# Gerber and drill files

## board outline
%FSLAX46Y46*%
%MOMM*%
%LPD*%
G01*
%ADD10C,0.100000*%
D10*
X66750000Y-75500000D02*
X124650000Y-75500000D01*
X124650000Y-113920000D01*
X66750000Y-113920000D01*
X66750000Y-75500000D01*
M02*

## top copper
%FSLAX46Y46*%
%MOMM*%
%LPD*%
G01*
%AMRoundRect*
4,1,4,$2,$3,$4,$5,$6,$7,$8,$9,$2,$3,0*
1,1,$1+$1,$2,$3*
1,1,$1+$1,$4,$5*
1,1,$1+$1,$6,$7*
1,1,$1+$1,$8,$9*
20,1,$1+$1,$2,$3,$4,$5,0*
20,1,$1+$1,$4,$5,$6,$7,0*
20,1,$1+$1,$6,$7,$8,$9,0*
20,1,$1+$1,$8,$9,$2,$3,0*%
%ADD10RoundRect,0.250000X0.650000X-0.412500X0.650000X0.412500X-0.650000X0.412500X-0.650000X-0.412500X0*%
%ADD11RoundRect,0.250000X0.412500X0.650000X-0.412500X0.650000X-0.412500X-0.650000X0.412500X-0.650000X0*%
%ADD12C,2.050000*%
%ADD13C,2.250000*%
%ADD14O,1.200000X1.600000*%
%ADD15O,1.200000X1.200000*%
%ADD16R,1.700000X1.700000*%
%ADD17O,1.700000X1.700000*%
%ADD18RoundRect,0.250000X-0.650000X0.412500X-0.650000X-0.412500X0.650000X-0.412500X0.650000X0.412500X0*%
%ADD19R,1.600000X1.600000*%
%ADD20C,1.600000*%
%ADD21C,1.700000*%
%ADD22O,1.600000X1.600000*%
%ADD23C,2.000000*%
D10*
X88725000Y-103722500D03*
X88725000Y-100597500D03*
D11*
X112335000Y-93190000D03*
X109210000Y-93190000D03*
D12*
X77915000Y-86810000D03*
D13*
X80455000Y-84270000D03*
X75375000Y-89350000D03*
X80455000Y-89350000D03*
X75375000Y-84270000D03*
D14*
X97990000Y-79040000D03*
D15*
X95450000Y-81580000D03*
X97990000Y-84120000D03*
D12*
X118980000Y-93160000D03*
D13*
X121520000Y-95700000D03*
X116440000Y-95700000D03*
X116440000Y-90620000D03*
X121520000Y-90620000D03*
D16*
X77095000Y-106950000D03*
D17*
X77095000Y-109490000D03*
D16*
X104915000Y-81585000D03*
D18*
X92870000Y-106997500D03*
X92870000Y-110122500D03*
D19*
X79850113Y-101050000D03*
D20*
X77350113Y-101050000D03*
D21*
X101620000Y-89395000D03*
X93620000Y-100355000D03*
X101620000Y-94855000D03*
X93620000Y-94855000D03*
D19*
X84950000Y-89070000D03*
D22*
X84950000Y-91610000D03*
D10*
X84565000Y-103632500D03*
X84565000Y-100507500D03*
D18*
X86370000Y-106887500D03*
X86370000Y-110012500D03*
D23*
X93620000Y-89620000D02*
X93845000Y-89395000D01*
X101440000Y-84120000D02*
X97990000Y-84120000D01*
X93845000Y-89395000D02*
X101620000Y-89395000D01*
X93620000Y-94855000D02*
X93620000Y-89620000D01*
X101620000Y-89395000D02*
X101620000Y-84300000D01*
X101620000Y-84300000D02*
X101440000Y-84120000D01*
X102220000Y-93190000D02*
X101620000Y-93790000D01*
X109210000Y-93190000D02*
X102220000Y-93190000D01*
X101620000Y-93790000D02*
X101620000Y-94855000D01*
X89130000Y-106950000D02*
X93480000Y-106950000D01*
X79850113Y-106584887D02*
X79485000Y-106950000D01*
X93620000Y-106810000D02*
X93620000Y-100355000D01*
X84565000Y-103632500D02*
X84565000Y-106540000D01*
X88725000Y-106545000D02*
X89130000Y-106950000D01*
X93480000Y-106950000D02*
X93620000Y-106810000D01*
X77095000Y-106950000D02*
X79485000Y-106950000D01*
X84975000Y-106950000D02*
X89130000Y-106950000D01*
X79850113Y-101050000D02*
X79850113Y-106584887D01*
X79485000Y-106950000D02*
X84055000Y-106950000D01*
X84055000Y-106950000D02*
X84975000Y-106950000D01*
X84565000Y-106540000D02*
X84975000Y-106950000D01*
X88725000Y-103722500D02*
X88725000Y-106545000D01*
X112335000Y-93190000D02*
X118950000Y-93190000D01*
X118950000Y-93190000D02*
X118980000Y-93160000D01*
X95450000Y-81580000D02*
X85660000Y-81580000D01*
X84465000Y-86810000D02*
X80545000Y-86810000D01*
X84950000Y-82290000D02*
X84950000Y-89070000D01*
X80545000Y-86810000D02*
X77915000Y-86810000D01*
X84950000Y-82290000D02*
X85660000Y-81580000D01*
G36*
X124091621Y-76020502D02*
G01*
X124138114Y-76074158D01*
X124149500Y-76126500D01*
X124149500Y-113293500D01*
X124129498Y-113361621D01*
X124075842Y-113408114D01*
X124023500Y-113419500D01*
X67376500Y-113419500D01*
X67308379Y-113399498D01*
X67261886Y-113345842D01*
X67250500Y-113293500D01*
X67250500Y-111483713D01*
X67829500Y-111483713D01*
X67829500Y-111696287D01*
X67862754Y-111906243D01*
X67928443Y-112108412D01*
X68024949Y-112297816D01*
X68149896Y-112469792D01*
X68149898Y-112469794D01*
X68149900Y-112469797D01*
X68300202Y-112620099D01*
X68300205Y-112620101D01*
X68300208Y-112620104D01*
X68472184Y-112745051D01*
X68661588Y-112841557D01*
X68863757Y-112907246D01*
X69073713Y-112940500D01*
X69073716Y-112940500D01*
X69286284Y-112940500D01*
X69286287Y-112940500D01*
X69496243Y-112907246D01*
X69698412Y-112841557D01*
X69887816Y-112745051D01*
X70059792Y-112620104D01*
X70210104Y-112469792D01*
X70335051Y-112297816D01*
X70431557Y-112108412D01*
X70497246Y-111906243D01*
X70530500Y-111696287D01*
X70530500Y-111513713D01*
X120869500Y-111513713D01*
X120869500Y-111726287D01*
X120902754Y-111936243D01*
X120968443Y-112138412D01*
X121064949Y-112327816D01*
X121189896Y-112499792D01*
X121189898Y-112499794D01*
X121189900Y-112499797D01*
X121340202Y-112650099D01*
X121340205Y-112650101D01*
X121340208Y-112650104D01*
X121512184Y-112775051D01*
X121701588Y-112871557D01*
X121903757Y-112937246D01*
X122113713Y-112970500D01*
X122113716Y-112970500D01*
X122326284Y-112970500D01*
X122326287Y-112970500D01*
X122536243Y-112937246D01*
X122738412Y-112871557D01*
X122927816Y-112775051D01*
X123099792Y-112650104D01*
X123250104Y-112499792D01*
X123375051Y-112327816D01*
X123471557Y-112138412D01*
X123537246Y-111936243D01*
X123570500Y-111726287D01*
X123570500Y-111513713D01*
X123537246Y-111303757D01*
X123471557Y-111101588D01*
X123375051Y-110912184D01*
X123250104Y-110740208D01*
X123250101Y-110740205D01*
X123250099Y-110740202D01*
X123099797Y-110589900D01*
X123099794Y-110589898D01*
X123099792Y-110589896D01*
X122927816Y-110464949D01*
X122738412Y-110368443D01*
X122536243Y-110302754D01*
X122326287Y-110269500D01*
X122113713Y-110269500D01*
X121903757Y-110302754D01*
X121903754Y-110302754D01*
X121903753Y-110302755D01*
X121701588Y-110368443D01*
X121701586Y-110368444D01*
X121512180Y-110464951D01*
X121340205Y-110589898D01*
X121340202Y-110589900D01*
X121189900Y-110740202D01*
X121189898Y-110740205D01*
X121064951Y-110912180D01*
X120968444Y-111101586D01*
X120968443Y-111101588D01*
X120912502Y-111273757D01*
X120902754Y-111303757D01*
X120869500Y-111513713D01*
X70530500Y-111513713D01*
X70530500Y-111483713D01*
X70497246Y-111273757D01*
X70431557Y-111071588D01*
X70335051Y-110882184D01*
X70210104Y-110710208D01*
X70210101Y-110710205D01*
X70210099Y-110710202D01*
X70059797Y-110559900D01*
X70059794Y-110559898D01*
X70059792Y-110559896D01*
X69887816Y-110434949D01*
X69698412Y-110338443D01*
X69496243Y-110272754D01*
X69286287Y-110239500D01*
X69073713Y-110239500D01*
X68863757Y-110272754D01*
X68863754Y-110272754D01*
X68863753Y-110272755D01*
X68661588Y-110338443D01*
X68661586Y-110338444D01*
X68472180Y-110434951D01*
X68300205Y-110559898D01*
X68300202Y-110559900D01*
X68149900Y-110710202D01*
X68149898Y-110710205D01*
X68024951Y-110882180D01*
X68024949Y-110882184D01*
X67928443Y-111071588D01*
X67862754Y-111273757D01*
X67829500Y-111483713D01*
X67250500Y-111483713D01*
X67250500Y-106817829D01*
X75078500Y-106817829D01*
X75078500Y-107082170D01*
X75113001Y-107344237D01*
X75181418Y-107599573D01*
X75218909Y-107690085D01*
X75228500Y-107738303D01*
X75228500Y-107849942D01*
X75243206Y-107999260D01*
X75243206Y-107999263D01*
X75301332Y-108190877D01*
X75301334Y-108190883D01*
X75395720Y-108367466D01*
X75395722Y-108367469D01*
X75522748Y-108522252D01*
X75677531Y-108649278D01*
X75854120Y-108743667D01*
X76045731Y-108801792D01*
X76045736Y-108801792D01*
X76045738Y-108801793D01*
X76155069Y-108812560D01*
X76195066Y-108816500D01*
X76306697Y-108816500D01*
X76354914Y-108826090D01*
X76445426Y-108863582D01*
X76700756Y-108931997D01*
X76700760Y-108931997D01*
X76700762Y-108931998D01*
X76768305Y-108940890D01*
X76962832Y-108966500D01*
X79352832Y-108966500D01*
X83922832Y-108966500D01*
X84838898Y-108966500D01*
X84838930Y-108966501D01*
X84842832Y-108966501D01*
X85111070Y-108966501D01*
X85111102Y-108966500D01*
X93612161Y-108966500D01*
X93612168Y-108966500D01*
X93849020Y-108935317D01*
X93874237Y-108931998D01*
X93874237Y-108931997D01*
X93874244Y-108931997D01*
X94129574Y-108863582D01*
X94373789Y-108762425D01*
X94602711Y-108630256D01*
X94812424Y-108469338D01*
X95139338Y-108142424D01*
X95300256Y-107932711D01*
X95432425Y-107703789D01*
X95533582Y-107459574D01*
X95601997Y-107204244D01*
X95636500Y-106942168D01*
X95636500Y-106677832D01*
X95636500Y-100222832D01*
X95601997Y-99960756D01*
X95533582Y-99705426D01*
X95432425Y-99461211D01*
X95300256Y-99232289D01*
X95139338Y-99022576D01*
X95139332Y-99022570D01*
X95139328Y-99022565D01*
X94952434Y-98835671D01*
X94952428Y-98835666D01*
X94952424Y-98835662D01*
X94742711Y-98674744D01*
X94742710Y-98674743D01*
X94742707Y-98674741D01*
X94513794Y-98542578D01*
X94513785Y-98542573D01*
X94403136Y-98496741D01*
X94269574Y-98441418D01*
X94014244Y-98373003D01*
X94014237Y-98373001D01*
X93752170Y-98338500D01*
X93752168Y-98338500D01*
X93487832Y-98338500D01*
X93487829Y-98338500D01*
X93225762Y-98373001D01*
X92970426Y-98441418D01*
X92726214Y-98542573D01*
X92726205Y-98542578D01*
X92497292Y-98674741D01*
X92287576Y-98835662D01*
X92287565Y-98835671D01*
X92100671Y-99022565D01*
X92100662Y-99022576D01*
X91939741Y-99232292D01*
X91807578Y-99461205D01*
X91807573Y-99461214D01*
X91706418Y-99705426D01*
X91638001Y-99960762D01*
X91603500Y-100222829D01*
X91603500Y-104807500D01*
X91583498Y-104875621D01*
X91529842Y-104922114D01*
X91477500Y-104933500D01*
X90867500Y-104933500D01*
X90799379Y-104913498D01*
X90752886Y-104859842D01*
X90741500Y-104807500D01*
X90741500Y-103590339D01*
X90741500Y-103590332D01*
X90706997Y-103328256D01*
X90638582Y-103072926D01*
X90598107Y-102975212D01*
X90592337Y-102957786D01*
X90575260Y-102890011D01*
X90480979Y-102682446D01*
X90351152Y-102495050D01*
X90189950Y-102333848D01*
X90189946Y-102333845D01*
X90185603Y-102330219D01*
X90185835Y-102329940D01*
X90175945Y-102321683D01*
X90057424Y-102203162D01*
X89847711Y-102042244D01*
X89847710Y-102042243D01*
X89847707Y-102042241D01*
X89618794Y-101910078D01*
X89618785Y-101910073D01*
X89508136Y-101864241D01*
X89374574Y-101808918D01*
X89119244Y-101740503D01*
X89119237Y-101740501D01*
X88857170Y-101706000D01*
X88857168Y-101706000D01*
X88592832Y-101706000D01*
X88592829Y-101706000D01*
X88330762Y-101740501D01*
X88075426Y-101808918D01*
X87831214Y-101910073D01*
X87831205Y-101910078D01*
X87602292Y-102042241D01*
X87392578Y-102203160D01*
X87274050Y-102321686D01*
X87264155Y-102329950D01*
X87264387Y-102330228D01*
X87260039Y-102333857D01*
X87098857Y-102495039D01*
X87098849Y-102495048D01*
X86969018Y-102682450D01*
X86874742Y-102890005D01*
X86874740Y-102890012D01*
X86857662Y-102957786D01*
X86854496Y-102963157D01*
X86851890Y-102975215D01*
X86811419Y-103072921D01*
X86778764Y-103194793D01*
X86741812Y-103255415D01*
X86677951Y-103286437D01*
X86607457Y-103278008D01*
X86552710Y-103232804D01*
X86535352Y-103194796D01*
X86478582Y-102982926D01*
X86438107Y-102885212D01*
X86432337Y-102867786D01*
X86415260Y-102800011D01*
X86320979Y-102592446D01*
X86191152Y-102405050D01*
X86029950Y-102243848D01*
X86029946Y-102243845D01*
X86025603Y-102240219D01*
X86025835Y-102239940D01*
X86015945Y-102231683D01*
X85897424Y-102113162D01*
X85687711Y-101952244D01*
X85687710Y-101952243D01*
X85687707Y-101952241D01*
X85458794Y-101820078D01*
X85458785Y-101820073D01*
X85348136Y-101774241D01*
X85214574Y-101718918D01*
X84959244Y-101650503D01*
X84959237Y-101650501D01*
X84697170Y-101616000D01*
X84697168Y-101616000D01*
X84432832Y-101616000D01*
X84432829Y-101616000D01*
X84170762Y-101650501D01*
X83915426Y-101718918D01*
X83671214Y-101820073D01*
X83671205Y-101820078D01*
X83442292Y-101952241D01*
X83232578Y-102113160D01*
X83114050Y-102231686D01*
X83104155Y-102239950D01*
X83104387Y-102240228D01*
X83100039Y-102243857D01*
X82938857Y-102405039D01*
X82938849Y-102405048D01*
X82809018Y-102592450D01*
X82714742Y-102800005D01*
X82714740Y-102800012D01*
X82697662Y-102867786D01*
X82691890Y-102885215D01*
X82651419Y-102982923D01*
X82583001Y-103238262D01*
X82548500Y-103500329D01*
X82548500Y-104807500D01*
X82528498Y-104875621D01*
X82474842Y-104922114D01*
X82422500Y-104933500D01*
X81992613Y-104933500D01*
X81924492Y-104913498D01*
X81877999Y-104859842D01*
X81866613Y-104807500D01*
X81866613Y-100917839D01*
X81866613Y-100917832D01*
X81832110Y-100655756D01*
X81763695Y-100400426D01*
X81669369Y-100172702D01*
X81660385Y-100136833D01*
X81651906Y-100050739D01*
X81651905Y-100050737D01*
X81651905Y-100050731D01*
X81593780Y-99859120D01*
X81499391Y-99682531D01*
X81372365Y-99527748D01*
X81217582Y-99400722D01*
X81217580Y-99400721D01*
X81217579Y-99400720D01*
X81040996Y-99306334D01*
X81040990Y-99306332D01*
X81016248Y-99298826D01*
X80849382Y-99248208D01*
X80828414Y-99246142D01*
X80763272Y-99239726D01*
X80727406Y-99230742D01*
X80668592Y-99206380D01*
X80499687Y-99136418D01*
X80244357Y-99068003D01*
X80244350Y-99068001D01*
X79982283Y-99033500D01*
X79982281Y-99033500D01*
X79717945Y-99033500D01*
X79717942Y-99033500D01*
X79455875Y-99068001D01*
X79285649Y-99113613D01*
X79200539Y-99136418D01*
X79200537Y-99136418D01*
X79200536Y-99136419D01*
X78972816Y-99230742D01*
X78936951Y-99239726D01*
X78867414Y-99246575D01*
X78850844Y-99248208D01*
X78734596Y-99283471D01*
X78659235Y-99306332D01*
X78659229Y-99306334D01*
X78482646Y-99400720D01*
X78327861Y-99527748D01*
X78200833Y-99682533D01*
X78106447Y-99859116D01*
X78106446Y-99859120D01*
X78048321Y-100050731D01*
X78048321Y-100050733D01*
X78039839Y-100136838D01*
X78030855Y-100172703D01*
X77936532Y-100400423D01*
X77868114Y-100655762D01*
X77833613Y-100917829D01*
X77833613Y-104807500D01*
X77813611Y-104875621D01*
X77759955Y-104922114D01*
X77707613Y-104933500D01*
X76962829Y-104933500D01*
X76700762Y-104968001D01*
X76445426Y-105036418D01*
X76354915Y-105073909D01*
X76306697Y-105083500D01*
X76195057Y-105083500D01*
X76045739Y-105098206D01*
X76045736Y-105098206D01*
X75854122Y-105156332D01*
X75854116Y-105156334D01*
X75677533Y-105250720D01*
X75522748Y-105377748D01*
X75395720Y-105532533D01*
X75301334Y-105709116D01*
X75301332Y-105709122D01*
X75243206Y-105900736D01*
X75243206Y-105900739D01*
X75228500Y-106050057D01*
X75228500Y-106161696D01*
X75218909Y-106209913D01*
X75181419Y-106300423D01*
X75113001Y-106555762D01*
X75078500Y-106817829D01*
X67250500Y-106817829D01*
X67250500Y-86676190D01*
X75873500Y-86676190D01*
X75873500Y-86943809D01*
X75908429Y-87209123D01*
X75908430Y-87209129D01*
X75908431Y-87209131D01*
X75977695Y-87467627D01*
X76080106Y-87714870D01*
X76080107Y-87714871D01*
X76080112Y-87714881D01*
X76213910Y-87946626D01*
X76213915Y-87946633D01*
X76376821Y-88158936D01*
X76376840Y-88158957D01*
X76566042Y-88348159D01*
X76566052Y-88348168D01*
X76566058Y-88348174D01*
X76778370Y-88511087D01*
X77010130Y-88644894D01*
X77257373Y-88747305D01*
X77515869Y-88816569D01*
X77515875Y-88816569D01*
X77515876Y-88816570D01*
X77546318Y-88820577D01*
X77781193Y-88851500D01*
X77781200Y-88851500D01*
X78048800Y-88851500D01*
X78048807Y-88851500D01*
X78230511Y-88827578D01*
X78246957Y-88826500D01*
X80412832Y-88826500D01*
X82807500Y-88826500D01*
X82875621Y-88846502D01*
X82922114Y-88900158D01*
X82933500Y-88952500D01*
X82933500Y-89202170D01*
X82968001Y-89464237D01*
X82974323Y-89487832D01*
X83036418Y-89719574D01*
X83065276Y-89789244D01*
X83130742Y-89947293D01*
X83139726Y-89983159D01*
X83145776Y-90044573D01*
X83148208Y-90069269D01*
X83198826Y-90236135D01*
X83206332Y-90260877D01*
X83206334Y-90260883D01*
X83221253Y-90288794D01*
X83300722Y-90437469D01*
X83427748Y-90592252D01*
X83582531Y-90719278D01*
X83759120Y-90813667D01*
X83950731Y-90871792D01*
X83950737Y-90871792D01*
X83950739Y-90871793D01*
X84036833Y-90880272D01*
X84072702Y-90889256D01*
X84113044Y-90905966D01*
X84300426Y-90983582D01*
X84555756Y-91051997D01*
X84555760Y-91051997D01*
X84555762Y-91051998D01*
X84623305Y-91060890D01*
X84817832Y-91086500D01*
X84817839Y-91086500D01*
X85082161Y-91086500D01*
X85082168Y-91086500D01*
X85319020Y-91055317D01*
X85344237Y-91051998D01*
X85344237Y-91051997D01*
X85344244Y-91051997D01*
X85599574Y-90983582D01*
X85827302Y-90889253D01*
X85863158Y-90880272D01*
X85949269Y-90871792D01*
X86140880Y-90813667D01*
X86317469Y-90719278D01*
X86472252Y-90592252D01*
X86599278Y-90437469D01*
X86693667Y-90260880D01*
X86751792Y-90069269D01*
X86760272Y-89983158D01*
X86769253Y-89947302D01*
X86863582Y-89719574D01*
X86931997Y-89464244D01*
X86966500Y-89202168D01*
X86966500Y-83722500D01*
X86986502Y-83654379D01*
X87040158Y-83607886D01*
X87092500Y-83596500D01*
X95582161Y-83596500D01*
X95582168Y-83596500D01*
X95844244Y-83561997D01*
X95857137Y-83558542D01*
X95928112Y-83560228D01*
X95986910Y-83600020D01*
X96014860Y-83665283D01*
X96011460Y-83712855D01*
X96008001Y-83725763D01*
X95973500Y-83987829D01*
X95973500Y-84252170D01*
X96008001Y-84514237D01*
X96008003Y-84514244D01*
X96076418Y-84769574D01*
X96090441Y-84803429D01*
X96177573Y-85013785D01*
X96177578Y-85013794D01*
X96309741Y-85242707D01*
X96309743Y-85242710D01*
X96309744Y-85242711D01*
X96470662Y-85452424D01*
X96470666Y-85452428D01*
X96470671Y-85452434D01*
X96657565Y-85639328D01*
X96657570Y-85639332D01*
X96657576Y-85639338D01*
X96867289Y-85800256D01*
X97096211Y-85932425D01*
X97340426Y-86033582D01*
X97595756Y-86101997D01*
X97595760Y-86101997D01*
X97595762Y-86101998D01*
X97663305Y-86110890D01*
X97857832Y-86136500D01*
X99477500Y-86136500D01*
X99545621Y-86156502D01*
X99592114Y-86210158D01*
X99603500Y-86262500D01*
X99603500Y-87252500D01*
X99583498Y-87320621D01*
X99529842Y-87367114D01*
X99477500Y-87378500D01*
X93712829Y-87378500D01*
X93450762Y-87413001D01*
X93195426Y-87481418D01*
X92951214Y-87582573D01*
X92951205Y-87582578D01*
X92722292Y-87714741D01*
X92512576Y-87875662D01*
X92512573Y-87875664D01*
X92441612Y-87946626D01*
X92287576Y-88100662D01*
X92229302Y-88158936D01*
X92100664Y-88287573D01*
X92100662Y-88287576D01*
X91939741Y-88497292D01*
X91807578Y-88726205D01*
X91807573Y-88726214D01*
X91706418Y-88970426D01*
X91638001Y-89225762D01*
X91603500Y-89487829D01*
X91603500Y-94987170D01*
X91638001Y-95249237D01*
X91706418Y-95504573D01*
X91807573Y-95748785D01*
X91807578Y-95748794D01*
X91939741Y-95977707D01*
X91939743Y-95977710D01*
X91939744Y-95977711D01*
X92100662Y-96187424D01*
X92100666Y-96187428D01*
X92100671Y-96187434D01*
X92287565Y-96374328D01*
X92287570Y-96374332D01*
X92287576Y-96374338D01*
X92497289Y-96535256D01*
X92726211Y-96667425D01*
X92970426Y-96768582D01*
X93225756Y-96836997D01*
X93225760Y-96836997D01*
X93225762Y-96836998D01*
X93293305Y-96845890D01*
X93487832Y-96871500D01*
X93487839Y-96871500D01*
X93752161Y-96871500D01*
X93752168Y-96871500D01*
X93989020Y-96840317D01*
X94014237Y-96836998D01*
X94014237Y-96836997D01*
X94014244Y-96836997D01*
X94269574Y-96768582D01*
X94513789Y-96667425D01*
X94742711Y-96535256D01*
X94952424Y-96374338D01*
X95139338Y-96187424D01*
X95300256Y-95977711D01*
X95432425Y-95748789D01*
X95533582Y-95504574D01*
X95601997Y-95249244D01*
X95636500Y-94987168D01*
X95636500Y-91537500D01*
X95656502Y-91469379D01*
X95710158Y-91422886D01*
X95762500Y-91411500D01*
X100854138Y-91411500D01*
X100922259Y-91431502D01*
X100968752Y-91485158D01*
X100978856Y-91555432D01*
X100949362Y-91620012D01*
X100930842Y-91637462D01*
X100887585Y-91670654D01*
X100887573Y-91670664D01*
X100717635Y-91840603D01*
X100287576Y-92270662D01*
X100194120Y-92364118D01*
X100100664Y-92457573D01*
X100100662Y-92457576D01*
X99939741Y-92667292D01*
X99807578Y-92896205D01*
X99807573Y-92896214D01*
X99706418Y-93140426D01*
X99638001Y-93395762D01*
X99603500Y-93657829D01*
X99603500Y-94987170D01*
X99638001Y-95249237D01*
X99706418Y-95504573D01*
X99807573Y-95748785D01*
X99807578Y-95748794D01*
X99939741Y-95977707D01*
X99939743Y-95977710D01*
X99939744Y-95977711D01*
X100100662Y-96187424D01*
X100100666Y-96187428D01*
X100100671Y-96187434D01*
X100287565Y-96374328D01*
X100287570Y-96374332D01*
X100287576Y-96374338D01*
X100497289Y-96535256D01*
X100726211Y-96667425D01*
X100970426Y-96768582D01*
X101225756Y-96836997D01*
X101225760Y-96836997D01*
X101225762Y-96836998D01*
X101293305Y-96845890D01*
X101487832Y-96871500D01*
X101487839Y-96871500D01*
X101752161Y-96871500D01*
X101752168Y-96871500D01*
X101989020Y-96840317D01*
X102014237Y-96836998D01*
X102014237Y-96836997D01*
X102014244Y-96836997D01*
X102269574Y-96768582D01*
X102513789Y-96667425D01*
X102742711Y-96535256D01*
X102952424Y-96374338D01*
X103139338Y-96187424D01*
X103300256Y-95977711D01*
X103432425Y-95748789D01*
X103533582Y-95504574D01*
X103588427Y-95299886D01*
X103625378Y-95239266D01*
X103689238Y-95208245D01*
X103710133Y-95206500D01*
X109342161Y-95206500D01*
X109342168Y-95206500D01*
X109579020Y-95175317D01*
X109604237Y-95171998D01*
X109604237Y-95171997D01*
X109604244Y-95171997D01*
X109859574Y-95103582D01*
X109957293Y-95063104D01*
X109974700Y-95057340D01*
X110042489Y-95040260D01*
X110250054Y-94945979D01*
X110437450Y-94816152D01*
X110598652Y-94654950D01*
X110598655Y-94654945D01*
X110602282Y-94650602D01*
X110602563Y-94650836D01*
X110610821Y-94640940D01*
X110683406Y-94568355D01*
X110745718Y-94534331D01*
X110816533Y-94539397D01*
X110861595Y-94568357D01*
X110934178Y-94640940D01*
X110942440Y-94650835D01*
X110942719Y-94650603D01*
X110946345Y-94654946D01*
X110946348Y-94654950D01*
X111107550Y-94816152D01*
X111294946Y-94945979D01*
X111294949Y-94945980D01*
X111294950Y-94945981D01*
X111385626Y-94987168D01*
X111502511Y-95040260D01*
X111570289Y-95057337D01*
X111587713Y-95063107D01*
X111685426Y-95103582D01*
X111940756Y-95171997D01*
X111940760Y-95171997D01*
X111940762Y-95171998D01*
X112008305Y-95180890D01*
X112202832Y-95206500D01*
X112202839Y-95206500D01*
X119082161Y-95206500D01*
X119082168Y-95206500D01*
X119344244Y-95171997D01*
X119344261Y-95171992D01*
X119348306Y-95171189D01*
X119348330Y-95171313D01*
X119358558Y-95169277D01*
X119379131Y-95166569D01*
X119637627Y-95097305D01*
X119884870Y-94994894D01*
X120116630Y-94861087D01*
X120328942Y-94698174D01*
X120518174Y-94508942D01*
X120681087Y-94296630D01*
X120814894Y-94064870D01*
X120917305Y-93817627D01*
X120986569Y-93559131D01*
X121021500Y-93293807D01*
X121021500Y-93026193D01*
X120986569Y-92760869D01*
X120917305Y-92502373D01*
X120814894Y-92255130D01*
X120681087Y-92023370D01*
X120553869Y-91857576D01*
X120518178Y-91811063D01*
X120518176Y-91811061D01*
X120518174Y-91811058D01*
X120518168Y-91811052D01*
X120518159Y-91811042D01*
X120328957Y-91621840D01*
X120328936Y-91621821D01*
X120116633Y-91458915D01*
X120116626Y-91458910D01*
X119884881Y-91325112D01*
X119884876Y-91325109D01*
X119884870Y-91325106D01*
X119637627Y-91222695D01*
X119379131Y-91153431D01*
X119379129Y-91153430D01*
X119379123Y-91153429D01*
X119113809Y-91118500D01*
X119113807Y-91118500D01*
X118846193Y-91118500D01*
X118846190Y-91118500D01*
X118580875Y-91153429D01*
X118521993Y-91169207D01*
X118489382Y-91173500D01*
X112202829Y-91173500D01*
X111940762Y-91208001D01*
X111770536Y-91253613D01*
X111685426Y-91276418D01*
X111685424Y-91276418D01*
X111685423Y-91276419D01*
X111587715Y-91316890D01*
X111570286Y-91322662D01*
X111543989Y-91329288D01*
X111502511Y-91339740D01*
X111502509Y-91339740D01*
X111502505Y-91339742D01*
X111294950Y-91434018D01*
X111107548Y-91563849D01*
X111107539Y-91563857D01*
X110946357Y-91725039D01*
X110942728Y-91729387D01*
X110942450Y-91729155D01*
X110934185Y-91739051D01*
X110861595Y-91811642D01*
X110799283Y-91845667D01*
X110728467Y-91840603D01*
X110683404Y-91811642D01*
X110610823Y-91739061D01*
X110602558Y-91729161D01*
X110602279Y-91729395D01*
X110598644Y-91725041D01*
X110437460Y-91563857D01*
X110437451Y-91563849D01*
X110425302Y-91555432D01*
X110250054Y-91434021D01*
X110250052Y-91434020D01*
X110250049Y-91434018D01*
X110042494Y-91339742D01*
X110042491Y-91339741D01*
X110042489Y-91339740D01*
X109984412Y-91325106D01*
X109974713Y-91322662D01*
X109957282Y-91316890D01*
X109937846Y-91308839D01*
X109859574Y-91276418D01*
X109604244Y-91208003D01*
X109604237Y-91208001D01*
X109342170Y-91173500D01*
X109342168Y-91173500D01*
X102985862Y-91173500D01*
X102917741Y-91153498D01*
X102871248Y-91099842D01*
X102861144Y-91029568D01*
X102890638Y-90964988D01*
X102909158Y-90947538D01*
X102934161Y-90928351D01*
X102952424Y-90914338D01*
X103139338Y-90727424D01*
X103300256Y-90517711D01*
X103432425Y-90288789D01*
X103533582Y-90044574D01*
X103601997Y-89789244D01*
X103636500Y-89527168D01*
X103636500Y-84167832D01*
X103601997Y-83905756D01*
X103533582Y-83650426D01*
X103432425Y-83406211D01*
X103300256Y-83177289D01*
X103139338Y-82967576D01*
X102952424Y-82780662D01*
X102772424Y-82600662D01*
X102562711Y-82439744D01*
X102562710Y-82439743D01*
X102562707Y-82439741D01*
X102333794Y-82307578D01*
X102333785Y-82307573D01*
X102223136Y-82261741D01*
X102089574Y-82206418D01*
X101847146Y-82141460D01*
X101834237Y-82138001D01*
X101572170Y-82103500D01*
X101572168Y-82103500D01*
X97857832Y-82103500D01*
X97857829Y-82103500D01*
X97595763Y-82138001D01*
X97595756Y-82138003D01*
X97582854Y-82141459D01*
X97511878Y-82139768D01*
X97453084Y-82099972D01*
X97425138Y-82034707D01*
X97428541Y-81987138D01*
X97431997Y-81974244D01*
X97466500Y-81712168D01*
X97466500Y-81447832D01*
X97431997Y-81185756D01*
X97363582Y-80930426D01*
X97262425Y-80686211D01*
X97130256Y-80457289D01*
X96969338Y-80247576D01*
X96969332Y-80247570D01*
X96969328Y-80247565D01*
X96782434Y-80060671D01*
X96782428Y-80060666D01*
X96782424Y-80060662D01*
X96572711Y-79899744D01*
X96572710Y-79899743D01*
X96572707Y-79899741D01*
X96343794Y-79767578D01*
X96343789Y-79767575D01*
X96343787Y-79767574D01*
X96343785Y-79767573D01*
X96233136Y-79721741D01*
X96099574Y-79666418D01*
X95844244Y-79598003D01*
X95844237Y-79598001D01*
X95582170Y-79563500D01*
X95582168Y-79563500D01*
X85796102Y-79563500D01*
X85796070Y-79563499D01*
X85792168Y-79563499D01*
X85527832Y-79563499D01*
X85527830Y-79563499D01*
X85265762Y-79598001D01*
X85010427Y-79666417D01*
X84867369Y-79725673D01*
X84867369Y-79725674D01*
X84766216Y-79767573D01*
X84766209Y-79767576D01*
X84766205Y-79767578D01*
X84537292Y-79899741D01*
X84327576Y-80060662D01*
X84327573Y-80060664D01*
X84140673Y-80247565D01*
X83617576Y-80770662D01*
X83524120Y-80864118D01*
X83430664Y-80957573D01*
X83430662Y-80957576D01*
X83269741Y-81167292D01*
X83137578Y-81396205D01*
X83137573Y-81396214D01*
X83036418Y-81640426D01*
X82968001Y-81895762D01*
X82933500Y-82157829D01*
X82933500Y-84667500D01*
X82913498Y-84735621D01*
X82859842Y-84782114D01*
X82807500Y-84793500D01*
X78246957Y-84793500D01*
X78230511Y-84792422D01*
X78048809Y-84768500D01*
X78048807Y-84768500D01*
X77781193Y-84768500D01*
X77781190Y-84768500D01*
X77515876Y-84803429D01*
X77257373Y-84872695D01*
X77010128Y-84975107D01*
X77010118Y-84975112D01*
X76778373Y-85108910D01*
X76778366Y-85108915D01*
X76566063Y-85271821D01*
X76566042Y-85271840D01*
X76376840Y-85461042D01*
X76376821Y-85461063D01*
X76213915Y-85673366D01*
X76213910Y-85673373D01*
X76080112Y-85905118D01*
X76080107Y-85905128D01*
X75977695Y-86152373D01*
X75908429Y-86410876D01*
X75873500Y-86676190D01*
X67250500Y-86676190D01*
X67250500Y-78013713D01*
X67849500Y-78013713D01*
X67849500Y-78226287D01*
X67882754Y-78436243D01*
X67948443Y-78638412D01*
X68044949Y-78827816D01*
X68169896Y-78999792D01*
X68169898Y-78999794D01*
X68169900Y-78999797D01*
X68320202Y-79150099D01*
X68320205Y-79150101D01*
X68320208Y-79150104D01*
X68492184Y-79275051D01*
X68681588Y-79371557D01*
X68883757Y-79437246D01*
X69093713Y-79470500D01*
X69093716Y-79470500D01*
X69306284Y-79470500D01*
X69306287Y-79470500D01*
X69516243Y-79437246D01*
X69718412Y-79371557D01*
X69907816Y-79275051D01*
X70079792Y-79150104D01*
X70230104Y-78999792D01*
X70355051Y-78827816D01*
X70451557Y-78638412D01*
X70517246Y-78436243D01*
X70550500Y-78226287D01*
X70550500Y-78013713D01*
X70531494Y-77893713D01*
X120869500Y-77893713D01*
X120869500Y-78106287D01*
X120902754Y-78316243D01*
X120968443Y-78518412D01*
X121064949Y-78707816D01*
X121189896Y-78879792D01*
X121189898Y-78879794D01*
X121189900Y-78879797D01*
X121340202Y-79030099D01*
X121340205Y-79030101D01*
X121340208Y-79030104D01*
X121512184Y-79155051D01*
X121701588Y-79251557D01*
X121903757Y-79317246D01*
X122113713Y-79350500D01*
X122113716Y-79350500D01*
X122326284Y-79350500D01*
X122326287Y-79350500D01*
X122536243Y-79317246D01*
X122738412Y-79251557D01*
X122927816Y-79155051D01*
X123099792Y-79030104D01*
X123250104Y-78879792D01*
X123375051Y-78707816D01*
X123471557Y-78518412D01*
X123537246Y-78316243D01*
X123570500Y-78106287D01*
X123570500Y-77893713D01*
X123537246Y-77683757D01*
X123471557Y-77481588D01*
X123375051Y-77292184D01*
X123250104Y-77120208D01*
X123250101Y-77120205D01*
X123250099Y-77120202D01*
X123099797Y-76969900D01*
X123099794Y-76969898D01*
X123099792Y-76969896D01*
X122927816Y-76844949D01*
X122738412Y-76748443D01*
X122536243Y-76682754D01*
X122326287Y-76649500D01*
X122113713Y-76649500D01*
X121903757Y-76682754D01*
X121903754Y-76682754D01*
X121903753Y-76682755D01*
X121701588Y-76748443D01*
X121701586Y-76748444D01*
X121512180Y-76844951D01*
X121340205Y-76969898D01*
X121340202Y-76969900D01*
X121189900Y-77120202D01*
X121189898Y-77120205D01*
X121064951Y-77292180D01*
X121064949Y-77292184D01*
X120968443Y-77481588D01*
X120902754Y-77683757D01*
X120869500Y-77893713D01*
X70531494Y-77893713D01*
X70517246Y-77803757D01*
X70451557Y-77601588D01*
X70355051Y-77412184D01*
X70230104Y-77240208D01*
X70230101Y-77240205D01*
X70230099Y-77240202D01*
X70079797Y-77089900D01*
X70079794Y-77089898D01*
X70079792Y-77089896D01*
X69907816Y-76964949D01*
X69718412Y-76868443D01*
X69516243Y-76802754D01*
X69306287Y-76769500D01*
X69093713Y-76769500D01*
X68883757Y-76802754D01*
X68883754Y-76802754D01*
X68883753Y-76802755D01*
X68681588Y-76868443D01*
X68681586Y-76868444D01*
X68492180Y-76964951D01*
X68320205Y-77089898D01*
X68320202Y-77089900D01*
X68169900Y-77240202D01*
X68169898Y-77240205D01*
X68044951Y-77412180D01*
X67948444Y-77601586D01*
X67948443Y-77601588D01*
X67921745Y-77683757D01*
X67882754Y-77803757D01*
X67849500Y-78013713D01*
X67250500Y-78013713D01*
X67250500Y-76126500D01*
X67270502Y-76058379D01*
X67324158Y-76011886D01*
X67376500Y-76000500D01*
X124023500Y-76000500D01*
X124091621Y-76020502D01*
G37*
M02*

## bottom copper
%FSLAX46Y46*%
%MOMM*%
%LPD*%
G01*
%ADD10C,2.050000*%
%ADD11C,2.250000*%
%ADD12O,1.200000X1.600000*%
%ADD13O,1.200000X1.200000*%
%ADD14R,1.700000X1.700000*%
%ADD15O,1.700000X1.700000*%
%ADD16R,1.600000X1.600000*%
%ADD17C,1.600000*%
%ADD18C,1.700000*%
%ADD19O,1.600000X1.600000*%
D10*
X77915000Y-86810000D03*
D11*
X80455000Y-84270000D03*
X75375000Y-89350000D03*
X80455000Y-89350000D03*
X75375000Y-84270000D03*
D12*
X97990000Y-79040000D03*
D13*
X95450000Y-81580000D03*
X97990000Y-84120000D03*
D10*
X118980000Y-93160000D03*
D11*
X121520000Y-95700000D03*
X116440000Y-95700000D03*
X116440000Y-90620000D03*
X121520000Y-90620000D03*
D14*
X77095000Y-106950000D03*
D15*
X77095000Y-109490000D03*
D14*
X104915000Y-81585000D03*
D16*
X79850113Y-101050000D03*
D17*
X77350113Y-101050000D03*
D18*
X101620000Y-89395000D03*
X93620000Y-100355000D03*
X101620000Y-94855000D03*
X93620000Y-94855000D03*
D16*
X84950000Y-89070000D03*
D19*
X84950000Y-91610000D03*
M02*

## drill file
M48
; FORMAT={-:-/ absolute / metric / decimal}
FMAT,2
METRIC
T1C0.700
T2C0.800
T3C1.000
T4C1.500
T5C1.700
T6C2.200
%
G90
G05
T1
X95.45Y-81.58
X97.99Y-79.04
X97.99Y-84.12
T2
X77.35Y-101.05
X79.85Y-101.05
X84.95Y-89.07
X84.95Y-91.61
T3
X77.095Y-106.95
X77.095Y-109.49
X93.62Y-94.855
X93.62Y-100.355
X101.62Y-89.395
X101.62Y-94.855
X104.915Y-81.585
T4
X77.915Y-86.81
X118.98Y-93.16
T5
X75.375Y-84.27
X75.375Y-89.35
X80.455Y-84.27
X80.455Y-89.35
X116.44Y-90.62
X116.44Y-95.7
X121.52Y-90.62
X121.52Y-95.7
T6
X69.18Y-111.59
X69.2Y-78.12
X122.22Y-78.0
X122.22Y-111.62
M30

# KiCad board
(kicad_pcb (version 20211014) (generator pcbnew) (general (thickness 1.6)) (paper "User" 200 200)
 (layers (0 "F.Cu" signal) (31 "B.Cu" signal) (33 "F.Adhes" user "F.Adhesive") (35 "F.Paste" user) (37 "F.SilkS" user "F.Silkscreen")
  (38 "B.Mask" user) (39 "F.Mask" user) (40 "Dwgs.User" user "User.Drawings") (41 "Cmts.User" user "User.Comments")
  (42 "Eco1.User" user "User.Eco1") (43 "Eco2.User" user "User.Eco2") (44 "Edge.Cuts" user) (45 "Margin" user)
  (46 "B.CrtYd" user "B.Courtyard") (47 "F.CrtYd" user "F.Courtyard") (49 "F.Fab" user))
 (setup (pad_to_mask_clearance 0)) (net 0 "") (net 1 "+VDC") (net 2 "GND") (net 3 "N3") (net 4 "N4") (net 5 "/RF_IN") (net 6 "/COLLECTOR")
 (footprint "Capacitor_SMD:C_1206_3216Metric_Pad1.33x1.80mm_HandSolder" (layer "F.Cu") (at 88.725 102.16 90)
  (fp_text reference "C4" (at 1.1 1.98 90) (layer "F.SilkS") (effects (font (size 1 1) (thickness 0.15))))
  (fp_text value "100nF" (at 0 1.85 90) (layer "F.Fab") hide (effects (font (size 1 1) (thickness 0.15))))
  (pad "1" smd roundrect (at -1.5625 0 90) (size 1.325 1.8) (layers "F.Cu" "F.Paste" "F.Mask") (roundrect_rratio 0.188679) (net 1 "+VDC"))
  (pad "2" smd roundrect (at 1.5625 0 90) (size 1.325 1.8) (layers "F.Cu" "F.Paste" "F.Mask") (roundrect_rratio 0.188679) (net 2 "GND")))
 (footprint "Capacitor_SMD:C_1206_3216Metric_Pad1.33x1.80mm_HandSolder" (layer "F.Cu") (at 110.7725 93.19 180)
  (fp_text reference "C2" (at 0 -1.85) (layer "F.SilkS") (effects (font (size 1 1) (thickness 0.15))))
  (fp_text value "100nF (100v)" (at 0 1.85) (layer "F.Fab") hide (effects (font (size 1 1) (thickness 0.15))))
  (pad "1" smd roundrect (at -1.5625 0 180) (size 1.325 1.8) (layers "F.Cu" "F.Paste" "F.Mask") (roundrect_rratio 0.188679) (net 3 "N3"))
  (pad "2" smd roundrect (at 1.5625 0 180) (size 1.325 1.8) (layers "F.Cu" "F.Paste" "F.Mask") (roundrect_rratio 0.188679) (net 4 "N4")))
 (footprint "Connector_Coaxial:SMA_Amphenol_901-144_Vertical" (layer "F.Cu") (at 77.915 86.81 180)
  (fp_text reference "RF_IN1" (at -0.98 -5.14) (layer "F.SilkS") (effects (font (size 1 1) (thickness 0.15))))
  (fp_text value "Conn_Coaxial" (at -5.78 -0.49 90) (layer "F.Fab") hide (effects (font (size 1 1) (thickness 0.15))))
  (pad "1" thru_hole circle locked (at 0 0 180) (size 2.05 2.05) (drill 1.5) (layers *.Cu *.Mask) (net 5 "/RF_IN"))
  (pad "2" thru_hole circle locked (at -2.54 2.54 180) (size 2.25 2.25) (drill 1.7) (layers *.Cu *.Mask) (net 2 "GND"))
  (pad "2" thru_hole circle locked (at 2.54 -2.54 180) (size 2.25 2.25) (drill 1.7) (layers *.Cu *.Mask) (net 2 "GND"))
  (pad "2" thru_hole circle locked (at -2.54 -2.54 180) (size 2.25 2.25) (drill 1.7) (layers *.Cu *.Mask) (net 2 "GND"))
  (pad "2" thru_hole circle locked (at 2.54 2.54 180) (size 2.25 2.25) (drill 1.7) (layers *.Cu *.Mask) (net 2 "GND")))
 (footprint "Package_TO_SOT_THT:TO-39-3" (layer "F.Cu") (at 97.99 79.04 -90)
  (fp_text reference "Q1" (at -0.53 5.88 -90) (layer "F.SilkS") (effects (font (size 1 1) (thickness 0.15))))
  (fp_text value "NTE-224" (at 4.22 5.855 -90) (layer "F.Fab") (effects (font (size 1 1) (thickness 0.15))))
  (pad "1" thru_hole oval (at 0 0 270) (size 1.6 1.2) (drill 0.7) (layers *.Cu *.Mask) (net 2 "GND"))
  (pad "2" thru_hole oval (at 2.54 2.54 270) (size 1.2 1.2) (drill 0.7) (layers *.Cu *.Mask) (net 5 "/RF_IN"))
  (pad "3" thru_hole oval (at 5.08 0 270) (size 1.2 1.2) (drill 0.7) (layers *.Cu *.Mask) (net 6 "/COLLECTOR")))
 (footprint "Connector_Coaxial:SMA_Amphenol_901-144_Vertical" (layer "F.Cu") (at 118.98 93.16 -90)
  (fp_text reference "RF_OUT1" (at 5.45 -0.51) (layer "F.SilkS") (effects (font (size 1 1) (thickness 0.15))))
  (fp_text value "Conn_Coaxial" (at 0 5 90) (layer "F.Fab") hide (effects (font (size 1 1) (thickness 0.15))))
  (pad "1" thru_hole circle locked (at 0 0 270) (size 2.05 2.05) (drill 1.5) (layers *.Cu *.Mask) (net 3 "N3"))
  (pad "2" thru_hole circle locked (at 2.54 -2.54 270) (size 2.25 2.25) (drill 1.7) (layers *.Cu *.Mask) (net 2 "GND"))
  (pad "2" thru_hole circle locked (at 2.54 2.54 270) (size 2.25 2.25) (drill 1.7) (layers *.Cu *.Mask) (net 2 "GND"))
  (pad "2" thru_hole circle locked (at -2.54 2.54 270) (size 2.25 2.25) (drill 1.7) (layers *.Cu *.Mask) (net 2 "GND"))
  (pad "2" thru_hole circle locked (at -2.54 -2.54 270) (size 2.25 2.25) (drill 1.7) (layers *.Cu *.Mask) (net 2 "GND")))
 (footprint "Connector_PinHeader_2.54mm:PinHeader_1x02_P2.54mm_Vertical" (layer "F.Cu") (at 77.095 106.95)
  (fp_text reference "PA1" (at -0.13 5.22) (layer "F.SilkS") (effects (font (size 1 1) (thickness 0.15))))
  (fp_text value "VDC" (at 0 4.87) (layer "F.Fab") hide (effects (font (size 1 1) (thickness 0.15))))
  (pad "1" thru_hole rect locked (at 0 0) (size 1.7 1.7) (drill 1) (layers *.Cu *.Mask) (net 1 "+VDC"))
  (pad "2" thru_hole oval locked (at 0 2.54) (size 1.7 1.7) (drill 1) (layers *.Cu *.Mask) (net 2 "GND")))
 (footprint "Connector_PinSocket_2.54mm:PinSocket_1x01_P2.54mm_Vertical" (layer "F.Cu") (at 104.915 81.585 180)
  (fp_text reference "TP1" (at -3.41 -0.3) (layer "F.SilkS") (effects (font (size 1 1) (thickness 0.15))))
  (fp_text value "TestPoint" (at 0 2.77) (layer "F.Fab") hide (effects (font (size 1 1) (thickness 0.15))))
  (pad "1" thru_hole rect (at 0 0 180) (size 1.7 1.7) (drill 1) (layers *.Cu *.Mask) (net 2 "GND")))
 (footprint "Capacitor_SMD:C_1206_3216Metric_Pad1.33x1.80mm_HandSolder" (layer "F.Cu") (at 92.87 108.56 -90)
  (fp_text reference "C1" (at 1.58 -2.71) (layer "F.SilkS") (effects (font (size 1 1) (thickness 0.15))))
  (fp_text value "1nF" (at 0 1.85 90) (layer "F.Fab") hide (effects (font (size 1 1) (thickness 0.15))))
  (pad "1" smd roundrect (at -1.5625 0 270) (size 1.325 1.8) (layers "F.Cu" "F.Paste" "F.Mask") (roundrect_rratio 0.188679) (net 1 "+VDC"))
  (pad "2" smd roundrect (at 1.5625 0 270) (size 1.325 1.8) (layers "F.Cu" "F.Paste" "F.Mask") (roundrect_rratio 0.188679) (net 2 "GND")))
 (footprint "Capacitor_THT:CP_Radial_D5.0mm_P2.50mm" (layer "F.Cu") (at 79.850113 101.05 180)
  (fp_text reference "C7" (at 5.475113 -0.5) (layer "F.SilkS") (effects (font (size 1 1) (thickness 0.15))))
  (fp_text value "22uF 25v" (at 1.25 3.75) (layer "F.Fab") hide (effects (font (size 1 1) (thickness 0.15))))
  (pad "1" thru_hole rect locked (at 0 0 180) (size 1.6 1.6) (drill 0.8) (layers *.Cu *.Mask) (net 1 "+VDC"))
  (pad "2" thru_hole circle locked (at 2.5 0 180) (size 1.6 1.6) (drill 0.8) (layers *.Cu *.Mask) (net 2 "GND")))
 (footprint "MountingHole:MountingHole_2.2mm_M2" (layer "F.Cu") (at 122.22 78)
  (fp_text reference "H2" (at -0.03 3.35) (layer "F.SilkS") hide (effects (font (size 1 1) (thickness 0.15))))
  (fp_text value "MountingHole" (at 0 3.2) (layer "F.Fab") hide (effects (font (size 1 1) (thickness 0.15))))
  (pad "" np_thru_hole circle (at 0 0) (size 2.2 2.2) (drill 2.2) (layers *.Cu *.Mask)))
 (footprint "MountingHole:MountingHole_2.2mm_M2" (layer "F.Cu") (at 69.2 78.12)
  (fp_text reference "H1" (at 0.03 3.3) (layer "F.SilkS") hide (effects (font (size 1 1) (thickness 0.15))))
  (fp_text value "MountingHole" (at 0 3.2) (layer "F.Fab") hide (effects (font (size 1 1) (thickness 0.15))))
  (pad "" np_thru_hole circle (at 0 0) (size 2.2 2.2) (drill 2.2) (layers *.Cu *.Mask)))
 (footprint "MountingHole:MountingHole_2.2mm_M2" (layer "F.Cu") (at 122.22 111.62)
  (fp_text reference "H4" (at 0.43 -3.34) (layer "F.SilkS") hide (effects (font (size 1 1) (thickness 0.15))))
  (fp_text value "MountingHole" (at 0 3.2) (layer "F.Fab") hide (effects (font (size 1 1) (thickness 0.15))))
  (pad "" np_thru_hole circle (at 0 0) (size 2.2 2.2) (drill 2.2) (layers *.Cu *.Mask)))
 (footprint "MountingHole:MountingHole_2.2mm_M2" (layer "F.Cu") (at 69.18 111.59)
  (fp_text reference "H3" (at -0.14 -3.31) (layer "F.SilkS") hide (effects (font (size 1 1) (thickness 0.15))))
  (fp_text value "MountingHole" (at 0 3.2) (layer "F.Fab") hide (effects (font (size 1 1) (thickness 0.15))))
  (pad "" np_thru_hole circle (at 0 0) (size 2.2 2.2) (drill 2.2) (layers *.Cu *.Mask)))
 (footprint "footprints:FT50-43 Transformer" (layer "F.Cu") (at 97.62 86.855)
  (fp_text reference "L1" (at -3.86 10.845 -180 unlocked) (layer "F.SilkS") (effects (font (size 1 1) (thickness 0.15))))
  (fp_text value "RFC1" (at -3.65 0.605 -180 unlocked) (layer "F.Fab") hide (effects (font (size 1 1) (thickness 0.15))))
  (pad "1" thru_hole circle locked (at 4 2.54) (size 1.7 1.7) (drill 1) (layers *.Cu *.Mask) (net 6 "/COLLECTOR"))
  (pad "2" thru_hole circle locked (at -4 13.5) (size 1.7 1.7) (drill 1) (layers *.Cu *.Mask) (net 1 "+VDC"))
  (pad "3" thru_hole circle locked (at 4 8) (size 1.7 1.7) (drill 1) (layers *.Cu *.Mask) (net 4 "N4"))
  (pad "4" thru_hole circle locked (at -4 8) (size 1.7 1.7) (drill 1) (layers *.Cu *.Mask) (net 6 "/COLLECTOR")))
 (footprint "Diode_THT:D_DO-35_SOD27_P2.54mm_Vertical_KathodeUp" (layer "F.Cu") (at 84.95 89.07 -90)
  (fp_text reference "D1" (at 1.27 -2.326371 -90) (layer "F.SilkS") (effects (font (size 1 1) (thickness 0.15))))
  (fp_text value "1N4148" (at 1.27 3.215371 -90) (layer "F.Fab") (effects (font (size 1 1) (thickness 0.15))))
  (pad "1" thru_hole rect (at 0 0 270) (size 1.6 1.6) (drill 0.8) (layers *.Cu *.Mask) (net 5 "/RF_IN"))
  (pad "2" thru_hole oval (at 2.54 0 270) (size 1.6 1.6) (drill 0.8) (layers *.Cu *.Mask) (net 2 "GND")))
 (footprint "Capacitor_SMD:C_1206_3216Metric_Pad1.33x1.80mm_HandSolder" (layer "F.Cu") (at 84.565 102.07 90)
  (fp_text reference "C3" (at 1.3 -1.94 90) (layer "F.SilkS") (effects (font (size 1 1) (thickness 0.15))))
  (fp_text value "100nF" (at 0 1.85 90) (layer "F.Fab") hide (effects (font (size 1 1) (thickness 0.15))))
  (pad "1" smd roundrect (at -1.5625 0 90) (size 1.325 1.8) (layers "F.Cu" "F.Paste" "F.Mask") (roundrect_rratio 0.188679) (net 1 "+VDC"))
  (pad "2" smd roundrect (at 1.5625 0 90) (size 1.325 1.8) (layers "F.Cu" "F.Paste" "F.Mask") (roundrect_rratio 0.188679) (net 2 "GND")))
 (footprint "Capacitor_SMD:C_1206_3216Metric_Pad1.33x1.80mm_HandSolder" (layer "F.Cu") (at 86.37 108.45 -90)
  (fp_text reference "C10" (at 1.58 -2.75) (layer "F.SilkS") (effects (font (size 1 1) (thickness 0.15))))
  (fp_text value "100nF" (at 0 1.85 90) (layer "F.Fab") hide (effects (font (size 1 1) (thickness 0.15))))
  (pad "1" smd roundrect (at -1.5625 0 270) (size 1.325 1.8) (layers "F.Cu" "F.Paste" "F.Mask") (roundrect_rratio 0.188679) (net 1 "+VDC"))
  (pad "2" smd roundrect (at 1.5625 0 270) (size 1.325 1.8) (layers "F.Cu" "F.Paste" "F.Mask") (roundrect_rratio 0.188679) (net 2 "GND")))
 (gr_rect (start 66.75 75.5) (end 124.65 113.92) (layer "Edge.Cuts") (width 0.1) (fill none))
 (segment (start 93.62 89.62) (end 93.845 89.395) (width 2) (layer "F.Cu") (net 6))
 (segment (start 101.44 84.12) (end 97.99 84.12) (width 2) (layer "F.Cu") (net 6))
 (segment (start 93.845 89.395) (end 101.62 89.395) (width 2) (layer "F.Cu") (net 6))
 (segment (start 93.62 94.855) (end 93.62 89.62) (width 2) (layer "F.Cu") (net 6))
 (segment (start 101.62 89.395) (end 101.62 84.3) (width 2) (layer "F.Cu") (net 6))
 (segment (start 101.62 84.3) (end 101.44 84.12) (width 2) (layer "F.Cu") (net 6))
 (segment (start 102.22 93.19) (end 101.62 93.79) (width 2) (layer "F.Cu") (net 4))
 (segment (start 109.21 93.19) (end 102.22 93.19) (width 2) (layer "F.Cu") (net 4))
 (segment (start 101.62 93.79) (end 101.62 94.855) (width 2) (layer "F.Cu") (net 4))
 (segment (start 89.13 106.95) (end 93.48 106.95) (width 2) (layer "F.Cu") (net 1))
 (segment (start 79.850113 106.584887) (end 79.485 106.95) (width 2) (layer "F.Cu") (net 1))
 (segment (start 93.62 106.81) (end 93.62 100.355) (width 2) (layer "F.Cu") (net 1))
 (segment (start 84.565 103.6325) (end 84.565 106.54) (width 2) (layer "F.Cu") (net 1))
 (segment (start 88.725 106.545) (end 89.13 106.95) (width 2) (layer "F.Cu") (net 1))
 (segment (start 93.48 106.95) (end 93.62 106.81) (width 2) (layer "F.Cu") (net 1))
 (segment (start 77.095 106.95) (end 79.485 106.95) (width 2) (layer "F.Cu") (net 1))
 (segment (start 84.975 106.95) (end 89.13 106.95) (width 2) (layer "F.Cu") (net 1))
 (segment (start 79.850113 101.05) (end 79.850113 106.584887) (width 2) (layer "F.Cu") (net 1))
 (segment (start 79.485 106.95) (end 84.055 106.95) (width 2) (layer "F.Cu") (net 1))
 (segment (start 84.055 106.95) (end 84.975 106.95) (width 2) (layer "F.Cu") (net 1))
 (segment (start 84.565 106.54) (end 84.975 106.95) (width 2) (layer "F.Cu") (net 1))
 (segment (start 88.725 103.7225) (end 88.725 106.545) (width 2) (layer "F.Cu") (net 1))
 (segment (start 112.335 93.19) (end 118.95 93.19) (width 2) (layer "F.Cu") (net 3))
 (segment (start 118.95 93.19) (end 118.98 93.16) (width 2) (layer "F.Cu") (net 3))
 (segment (start 95.45 81.58) (end 85.66 81.58) (width 2) (layer "F.Cu") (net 5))
 (segment (start 84.465 86.81) (end 80.545 86.81) (width 2) (layer "F.Cu") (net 5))
 (segment (start 84.95 82.29) (end 84.95 89.07) (width 2) (layer "F.Cu") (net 5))
 (segment (start 80.545 86.81) (end 77.915 86.81) (width 2) (layer "F.Cu") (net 5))
 (segment (start 84.95 82.29) (end 85.66 81.58) (width 2) (layer "F.Cu") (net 5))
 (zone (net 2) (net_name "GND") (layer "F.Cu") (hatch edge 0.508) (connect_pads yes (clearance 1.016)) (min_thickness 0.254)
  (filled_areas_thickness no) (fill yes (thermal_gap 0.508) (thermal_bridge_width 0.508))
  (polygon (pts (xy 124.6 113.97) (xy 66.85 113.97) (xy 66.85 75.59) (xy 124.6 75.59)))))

